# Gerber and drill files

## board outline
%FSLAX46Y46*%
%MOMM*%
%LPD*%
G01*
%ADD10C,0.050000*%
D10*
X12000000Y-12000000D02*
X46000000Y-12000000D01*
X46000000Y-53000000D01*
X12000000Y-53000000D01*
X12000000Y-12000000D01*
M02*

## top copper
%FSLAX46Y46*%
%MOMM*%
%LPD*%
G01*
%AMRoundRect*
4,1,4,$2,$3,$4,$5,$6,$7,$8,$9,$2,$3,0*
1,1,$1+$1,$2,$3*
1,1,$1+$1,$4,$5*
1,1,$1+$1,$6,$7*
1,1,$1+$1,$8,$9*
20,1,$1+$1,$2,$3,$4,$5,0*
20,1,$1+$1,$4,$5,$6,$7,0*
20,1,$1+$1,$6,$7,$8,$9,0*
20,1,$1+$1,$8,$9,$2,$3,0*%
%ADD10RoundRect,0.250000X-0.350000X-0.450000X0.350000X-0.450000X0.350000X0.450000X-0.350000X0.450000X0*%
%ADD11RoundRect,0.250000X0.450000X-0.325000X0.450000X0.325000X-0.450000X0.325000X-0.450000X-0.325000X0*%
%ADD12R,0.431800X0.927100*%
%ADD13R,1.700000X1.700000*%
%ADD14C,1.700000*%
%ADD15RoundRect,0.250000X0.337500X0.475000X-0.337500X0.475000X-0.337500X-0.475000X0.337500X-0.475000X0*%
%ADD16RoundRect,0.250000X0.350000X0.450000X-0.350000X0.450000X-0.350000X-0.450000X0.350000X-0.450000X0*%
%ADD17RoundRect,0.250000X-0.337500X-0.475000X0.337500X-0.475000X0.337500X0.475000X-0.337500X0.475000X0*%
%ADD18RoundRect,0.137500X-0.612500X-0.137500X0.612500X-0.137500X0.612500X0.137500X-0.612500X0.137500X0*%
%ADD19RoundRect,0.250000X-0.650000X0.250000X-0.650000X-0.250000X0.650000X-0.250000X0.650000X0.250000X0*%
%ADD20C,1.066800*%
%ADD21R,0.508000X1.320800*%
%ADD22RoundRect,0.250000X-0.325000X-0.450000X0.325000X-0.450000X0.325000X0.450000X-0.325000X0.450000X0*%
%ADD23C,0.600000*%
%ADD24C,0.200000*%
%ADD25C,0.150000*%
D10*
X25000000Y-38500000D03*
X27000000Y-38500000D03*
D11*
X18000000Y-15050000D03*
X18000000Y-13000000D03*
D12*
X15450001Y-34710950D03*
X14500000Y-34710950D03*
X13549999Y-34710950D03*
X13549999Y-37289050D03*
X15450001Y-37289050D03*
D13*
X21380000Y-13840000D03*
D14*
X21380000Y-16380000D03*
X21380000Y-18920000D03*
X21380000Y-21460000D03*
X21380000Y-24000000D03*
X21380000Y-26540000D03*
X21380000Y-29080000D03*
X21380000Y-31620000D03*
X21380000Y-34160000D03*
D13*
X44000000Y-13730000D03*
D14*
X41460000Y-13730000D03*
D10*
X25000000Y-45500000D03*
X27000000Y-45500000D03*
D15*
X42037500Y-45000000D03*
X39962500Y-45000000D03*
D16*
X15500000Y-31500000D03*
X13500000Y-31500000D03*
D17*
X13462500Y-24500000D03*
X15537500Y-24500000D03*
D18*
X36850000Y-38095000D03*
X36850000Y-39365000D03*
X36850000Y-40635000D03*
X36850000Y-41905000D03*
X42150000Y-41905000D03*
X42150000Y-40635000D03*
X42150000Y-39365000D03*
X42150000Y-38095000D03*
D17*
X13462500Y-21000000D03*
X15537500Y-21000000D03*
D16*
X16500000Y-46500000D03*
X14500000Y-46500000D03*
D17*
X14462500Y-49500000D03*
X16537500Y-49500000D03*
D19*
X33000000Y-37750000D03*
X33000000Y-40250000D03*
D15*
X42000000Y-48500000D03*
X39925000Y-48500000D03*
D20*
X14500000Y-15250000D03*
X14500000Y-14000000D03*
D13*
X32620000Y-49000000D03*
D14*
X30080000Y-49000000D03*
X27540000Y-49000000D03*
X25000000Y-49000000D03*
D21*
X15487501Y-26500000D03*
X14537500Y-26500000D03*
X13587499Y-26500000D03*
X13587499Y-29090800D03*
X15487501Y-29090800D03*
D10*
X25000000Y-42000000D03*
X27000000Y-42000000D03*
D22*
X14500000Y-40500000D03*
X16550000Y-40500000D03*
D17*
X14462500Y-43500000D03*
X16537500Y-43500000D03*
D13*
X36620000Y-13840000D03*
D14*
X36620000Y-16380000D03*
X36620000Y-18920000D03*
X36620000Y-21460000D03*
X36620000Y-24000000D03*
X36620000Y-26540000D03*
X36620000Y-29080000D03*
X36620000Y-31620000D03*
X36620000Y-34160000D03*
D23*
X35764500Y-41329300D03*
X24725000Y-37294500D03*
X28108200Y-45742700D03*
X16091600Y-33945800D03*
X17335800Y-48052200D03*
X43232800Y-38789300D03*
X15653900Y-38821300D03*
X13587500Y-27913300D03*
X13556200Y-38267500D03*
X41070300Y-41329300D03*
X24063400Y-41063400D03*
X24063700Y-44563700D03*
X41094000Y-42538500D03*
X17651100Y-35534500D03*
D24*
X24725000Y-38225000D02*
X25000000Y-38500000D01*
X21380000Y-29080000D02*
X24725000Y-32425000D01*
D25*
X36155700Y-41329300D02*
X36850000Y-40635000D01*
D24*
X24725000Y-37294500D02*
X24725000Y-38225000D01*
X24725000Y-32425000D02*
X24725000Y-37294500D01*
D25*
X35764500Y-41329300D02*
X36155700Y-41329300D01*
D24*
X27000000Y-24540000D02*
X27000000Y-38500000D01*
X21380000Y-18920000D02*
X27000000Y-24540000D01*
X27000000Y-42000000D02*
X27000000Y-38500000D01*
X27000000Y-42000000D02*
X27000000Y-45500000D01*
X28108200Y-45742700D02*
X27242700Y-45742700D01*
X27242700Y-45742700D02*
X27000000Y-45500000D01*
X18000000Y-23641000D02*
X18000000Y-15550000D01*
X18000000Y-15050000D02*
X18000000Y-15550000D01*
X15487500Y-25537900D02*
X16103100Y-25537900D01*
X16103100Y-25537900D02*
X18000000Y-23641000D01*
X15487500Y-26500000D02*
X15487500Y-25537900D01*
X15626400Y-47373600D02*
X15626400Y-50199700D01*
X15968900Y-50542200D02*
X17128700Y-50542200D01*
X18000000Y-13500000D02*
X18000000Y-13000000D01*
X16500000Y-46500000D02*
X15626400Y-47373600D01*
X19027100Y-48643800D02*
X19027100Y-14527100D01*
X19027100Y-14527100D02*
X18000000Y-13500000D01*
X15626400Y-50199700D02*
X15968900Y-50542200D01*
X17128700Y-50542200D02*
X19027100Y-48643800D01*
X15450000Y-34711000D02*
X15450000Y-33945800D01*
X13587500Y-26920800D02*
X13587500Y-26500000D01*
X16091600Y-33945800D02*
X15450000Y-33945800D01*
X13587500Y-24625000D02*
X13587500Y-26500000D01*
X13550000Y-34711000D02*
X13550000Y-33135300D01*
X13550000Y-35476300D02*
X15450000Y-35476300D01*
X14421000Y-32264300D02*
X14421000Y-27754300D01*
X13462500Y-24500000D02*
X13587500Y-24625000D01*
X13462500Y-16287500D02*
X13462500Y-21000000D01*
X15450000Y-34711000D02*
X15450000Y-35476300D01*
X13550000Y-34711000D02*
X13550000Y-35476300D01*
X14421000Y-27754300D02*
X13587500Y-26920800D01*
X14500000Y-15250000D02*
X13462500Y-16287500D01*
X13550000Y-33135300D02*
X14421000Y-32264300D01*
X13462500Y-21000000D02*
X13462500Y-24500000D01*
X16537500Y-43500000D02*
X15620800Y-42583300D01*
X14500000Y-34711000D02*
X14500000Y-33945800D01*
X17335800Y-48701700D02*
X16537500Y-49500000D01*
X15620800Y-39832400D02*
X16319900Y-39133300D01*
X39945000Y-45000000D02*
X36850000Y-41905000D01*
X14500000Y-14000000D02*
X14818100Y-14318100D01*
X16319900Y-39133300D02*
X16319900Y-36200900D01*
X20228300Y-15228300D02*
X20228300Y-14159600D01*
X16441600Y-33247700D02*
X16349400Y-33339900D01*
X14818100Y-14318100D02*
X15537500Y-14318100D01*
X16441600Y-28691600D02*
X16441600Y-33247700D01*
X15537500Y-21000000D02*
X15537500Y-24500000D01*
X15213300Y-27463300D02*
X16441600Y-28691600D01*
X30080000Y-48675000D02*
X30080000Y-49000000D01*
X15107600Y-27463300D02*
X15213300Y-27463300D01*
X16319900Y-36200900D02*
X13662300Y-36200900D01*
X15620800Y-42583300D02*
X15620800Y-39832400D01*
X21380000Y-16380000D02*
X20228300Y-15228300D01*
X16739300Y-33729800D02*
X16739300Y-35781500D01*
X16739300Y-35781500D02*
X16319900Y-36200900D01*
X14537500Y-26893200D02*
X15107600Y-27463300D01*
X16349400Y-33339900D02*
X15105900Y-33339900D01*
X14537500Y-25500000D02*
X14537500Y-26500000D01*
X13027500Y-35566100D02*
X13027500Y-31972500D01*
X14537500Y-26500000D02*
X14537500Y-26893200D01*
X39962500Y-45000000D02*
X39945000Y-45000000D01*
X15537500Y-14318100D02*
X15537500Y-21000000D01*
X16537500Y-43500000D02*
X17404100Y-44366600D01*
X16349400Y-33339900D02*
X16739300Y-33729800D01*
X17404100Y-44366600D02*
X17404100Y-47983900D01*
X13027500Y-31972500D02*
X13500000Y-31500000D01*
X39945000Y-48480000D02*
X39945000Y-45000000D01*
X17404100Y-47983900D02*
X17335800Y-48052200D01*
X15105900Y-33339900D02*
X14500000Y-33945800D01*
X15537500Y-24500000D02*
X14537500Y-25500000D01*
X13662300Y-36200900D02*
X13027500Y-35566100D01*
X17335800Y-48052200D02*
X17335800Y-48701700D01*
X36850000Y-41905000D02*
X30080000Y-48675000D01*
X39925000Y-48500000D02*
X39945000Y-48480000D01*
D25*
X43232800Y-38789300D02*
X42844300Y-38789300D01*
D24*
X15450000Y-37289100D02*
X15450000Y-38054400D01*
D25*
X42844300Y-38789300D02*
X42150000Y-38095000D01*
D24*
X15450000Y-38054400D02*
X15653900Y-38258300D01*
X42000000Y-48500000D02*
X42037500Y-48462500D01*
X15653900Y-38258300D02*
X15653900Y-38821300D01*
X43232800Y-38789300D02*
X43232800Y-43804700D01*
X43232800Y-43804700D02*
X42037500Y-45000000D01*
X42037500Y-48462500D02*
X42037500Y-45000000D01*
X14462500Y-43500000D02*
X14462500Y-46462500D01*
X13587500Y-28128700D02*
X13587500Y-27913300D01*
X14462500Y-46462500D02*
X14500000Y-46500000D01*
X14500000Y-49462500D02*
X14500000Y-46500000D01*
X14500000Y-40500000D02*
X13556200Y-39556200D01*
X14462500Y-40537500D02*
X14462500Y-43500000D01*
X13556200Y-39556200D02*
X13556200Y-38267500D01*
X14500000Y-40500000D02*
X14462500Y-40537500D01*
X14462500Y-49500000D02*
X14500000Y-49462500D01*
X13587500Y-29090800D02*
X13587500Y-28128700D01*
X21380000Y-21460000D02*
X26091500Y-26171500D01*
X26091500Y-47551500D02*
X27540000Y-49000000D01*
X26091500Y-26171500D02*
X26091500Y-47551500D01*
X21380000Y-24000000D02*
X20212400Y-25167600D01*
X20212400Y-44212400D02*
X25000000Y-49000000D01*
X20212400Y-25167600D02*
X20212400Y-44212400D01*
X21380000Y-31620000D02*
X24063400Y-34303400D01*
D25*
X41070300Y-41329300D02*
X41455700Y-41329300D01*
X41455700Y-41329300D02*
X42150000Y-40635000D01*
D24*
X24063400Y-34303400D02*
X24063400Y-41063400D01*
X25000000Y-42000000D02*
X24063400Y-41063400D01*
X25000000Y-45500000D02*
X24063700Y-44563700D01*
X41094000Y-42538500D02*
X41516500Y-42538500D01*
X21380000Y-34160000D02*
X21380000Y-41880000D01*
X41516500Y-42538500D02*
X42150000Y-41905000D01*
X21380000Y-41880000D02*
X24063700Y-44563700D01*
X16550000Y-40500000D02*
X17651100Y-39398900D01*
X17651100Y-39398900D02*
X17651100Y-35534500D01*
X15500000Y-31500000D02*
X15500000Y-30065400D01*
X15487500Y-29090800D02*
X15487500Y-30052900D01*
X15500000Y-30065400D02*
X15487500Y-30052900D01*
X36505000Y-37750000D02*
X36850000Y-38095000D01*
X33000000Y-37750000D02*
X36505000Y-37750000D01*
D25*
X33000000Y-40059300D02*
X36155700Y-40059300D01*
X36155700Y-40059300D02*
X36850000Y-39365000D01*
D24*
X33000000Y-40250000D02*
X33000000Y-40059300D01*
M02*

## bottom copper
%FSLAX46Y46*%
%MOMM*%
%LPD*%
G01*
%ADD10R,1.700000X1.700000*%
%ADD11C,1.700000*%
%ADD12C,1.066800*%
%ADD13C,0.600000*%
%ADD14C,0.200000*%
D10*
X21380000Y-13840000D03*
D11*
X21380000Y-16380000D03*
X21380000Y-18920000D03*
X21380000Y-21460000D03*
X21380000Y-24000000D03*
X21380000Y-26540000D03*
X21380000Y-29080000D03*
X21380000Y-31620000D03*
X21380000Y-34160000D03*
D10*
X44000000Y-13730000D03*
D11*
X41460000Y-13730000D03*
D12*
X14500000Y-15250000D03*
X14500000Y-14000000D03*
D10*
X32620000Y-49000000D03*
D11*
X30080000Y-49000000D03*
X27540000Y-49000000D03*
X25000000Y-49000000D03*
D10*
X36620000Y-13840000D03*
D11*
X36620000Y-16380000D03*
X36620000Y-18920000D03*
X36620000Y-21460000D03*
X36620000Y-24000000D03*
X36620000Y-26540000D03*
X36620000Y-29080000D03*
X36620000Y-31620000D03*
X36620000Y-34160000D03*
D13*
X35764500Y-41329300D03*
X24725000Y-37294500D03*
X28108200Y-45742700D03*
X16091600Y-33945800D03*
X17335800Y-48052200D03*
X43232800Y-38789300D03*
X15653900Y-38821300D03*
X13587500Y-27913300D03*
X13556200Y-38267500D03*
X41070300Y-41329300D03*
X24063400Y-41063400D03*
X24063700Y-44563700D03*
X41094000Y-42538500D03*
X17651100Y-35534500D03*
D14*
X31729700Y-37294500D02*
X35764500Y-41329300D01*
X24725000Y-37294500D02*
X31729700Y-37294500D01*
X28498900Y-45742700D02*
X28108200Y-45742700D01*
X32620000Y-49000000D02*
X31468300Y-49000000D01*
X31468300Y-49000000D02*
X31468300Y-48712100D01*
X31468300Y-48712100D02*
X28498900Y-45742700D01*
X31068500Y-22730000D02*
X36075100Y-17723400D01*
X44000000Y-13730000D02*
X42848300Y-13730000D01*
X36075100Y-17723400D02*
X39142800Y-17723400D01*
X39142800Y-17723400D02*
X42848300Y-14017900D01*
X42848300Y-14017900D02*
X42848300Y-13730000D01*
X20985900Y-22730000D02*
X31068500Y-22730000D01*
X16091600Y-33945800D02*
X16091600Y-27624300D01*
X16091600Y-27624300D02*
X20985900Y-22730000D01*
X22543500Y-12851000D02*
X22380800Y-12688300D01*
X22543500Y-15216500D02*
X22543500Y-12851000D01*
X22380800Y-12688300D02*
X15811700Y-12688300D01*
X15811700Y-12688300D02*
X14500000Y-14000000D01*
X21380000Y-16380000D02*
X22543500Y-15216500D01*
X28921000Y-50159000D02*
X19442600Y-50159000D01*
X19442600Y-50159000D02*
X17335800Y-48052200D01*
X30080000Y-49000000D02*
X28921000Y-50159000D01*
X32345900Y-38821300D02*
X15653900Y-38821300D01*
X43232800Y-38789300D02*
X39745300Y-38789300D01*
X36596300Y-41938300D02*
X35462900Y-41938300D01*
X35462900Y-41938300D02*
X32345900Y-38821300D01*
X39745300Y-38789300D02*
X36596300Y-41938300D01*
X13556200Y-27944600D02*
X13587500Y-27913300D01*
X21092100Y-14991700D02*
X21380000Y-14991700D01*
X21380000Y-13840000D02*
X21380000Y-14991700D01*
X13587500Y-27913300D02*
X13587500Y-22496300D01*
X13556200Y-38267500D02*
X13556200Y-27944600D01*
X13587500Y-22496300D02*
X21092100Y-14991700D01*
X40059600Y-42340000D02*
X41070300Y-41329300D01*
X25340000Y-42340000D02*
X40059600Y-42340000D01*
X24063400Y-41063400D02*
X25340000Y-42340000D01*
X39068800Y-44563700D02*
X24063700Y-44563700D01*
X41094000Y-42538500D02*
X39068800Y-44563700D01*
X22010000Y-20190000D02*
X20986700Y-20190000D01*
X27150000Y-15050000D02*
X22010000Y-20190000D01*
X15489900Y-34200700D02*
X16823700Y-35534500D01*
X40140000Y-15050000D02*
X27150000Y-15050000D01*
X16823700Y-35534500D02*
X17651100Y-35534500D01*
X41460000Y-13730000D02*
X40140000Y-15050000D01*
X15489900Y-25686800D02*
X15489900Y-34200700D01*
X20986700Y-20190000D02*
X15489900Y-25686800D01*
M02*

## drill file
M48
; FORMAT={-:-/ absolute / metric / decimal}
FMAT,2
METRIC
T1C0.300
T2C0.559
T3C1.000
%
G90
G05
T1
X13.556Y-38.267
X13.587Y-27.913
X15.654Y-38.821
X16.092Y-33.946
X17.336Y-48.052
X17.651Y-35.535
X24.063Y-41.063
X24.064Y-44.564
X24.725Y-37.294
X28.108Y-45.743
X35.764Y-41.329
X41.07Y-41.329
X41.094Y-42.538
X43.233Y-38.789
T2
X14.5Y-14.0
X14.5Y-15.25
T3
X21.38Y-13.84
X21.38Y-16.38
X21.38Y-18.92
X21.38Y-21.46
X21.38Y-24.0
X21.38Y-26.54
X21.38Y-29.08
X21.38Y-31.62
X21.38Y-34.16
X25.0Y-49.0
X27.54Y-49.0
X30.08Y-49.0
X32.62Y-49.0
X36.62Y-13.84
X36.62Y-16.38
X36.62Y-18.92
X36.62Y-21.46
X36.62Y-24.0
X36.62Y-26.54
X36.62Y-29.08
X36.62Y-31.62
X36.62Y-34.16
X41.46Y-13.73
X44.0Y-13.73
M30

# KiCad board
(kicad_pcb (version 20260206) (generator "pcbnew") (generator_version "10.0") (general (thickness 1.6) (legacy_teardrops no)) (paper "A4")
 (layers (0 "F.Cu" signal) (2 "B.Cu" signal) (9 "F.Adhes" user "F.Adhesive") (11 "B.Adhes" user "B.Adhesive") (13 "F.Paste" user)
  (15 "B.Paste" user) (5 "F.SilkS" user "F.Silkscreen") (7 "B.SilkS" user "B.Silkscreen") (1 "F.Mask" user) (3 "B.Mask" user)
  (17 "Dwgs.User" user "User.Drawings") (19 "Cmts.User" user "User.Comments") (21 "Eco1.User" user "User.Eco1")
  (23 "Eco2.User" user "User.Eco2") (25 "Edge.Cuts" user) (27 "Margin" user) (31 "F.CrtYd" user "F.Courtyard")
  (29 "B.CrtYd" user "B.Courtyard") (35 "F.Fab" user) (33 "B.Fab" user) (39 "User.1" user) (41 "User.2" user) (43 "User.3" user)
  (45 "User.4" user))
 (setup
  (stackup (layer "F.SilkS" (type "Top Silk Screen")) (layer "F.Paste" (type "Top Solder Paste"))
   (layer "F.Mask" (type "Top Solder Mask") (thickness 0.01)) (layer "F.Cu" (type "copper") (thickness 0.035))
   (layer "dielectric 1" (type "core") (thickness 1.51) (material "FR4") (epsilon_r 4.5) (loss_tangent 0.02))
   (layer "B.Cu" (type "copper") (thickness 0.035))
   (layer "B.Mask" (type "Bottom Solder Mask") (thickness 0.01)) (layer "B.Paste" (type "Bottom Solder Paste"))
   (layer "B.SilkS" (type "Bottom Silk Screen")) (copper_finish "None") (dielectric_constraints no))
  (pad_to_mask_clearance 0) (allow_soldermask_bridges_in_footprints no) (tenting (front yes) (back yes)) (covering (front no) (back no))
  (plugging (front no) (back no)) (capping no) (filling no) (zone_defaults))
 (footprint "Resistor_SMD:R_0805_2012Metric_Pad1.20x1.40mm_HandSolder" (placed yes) (layer "F.Cu") (at 26 38.5)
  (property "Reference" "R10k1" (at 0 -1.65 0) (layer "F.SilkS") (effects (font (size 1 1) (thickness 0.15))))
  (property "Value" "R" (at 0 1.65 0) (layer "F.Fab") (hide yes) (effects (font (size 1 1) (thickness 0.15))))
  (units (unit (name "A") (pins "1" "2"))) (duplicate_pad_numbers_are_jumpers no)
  (pad "1" smd roundrect (at -1 0) (size 1.2 1.4) (layers "F.Cu" "F.Mask" "F.Paste") (roundrect_rratio 0.208333) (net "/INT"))
  (pad "2" smd roundrect (at 1 0) (size 1.2 1.4) (layers "F.Cu" "F.Mask" "F.Paste") (roundrect_rratio 0.208333) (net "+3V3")))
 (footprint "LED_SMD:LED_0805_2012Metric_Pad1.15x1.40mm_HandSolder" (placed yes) (layer "F.Cu") (at 18 14.025 90)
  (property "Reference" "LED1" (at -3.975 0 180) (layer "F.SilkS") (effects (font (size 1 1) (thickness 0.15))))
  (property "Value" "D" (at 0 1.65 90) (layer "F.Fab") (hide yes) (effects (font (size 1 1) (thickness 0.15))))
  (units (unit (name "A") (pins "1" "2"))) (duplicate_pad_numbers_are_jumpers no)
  (pad "1" smd roundrect (at -1.025 0 90) (size 1.15 1.4) (layers "F.Cu" "F.Mask" "F.Paste") (roundrect_rratio 0.217391) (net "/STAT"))
  (pad "2" smd roundrect (at 1.025 0 90) (size 1.15 1.4) (layers "F.Cu" "F.Mask" "F.Paste") (roundrect_rratio 0.217391) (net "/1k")))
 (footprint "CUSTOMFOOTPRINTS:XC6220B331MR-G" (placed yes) (layer "F.Cu") (at 14.5 36 -90)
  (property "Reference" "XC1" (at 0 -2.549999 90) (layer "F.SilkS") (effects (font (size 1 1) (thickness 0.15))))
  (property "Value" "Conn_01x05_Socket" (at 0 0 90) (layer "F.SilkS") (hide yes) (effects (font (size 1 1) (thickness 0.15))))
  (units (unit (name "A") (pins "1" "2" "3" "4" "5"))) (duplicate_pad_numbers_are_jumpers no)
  (pad "1" smd rect (at -1.28905 -0.950001 270) (size 0.9271 0.4318) (layers "F.Cu" "F.Mask" "F.Paste") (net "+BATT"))
  (pad "2" smd rect (at -1.28905 0 270) (size 0.9271 0.4318) (layers "F.Cu" "F.Mask" "F.Paste") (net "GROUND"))
  (pad "3" smd rect (at -1.28905 0.950001 270) (size 0.9271 0.4318) (layers "F.Cu" "F.Mask" "F.Paste") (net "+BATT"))
  (pad "4" smd rect (at 1.28905 0.950001 270) (size 0.9271 0.4318) (layers "F.Cu" "F.Mask" "F.Paste") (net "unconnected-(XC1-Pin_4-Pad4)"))
  (pad "5" smd rect (at 1.28905 -0.950001 270) (size 0.9271 0.4318) (layers "F.Cu" "F.Mask" "F.Paste") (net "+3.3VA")))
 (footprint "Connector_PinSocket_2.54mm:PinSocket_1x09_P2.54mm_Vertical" (layer "F.Cu") (at 21.38 13.84)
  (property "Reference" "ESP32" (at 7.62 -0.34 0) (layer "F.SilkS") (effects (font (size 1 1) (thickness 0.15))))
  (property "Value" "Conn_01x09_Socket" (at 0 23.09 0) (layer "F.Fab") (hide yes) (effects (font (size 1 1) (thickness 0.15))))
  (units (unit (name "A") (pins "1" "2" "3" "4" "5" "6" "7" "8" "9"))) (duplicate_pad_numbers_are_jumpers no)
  (pad "1" thru_hole rect (at 0 0) (size 1.7 1.7) (drill 1) (layers "*.Cu" "*.Mask") (remove_unused_layers no) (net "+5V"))
  (pad "2" thru_hole circle (at 0 2.54) (size 1.7 1.7) (drill 1) (layers "*.Cu" "*.Mask") (remove_unused_layers no) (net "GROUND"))
  (pad "3" thru_hole circle (at 0 5.08) (size 1.7 1.7) (drill 1) (layers "*.Cu" "*.Mask") (remove_unused_layers no) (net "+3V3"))
  (pad "4" thru_hole circle (at 0 7.62) (size 1.7 1.7) (drill 1) (layers "*.Cu" "*.Mask") (remove_unused_layers no) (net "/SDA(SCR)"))
  (pad "5" thru_hole circle (at 0 10.16) (size 1.7 1.7) (drill 1) (layers "*.Cu" "*.Mask") (remove_unused_layers no) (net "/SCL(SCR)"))
  (pad "6" thru_hole circle (at 0 12.7) (size 1.7 1.7) (drill 1) (layers "*.Cu" "*.Mask") (remove_unused_layers no)
   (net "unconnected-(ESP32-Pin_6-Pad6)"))
  (pad "7" thru_hole circle (at 0 15.24) (size 1.7 1.7) (drill 1) (layers "*.Cu" "*.Mask") (remove_unused_layers no) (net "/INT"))
  (pad "8" thru_hole circle (at 0 17.78) (size 1.7 1.7) (drill 1) (layers "*.Cu" "*.Mask") (remove_unused_layers no) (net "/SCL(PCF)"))
  (pad "9" thru_hole circle (at 0 20.32) (size 1.7 1.7) (drill 1) (layers "*.Cu" "*.Mask") (remove_unused_layers no) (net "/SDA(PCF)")))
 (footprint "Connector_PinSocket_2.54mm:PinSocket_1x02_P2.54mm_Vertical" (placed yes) (layer "F.Cu") (at 44 13.73 -90)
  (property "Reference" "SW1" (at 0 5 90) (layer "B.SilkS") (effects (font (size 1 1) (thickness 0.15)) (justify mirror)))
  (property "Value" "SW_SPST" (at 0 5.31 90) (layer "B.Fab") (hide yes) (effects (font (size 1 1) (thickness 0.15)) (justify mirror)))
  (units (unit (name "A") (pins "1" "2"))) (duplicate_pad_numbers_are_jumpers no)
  (pad "1" thru_hole rect (at 0 0 270) (size 1.7 1.7) (drill 1) (layers "*.Cu" "*.Mask") (remove_unused_layers no) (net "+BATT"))
  (pad "2" thru_hole circle (at 0 2.54 270) (size 1.7 1.7) (drill 1) (layers "*.Cu" "*.Mask") (remove_unused_layers no) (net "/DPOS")))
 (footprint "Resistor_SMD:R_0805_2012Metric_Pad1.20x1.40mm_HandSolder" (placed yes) (layer "F.Cu") (at 26 45.5)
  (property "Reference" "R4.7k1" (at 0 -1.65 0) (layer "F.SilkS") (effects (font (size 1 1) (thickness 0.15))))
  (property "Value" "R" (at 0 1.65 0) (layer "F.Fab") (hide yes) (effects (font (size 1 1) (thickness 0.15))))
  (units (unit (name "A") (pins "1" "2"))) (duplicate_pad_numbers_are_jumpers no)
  (pad "1" smd roundrect (at -1 0) (size 1.2 1.4) (layers "F.Cu" "F.Mask" "F.Paste") (roundrect_rratio 0.208333) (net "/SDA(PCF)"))
  (pad "2" smd roundrect (at 1 0) (size 1.2 1.4) (layers "F.Cu" "F.Mask" "F.Paste") (roundrect_rratio 0.208333) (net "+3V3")))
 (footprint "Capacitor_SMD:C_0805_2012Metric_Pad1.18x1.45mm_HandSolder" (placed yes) (layer "F.Cu") (at 41 45 180)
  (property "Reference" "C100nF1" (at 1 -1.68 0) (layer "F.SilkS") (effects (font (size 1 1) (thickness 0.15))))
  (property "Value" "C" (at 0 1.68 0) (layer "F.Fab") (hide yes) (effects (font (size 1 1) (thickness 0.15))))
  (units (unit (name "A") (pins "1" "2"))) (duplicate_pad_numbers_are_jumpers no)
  (pad "1" smd roundrect (at -1.0375 0 180) (size 1.175 1.45) (layers "F.Cu" "F.Mask" "F.Paste") (roundrect_rratio 0.212766) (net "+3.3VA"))
  (pad "2" smd roundrect (at 1.0375 0 180) (size 1.175 1.45) (layers "F.Cu" "F.Mask" "F.Paste") (roundrect_rratio 0.212766) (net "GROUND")))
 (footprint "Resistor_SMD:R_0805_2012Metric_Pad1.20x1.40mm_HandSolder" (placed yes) (layer "F.Cu") (at 14.5 31.5 180)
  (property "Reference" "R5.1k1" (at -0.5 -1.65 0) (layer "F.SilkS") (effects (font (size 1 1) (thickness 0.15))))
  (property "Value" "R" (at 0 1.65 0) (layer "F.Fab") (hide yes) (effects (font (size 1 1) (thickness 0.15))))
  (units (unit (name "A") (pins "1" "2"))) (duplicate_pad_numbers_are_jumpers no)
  (pad "1" smd roundrect (at -1 0 180) (size 1.2 1.4) (layers "F.Cu" "F.Mask" "F.Paste") (roundrect_rratio 0.208333) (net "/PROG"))
  (pad "2" smd roundrect (at 1 0 180) (size 1.2 1.4) (layers "F.Cu" "F.Mask" "F.Paste") (roundrect_rratio 0.208333) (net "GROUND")))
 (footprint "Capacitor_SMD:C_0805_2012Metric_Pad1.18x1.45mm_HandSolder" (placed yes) (layer "F.Cu") (at 14.5 24.5)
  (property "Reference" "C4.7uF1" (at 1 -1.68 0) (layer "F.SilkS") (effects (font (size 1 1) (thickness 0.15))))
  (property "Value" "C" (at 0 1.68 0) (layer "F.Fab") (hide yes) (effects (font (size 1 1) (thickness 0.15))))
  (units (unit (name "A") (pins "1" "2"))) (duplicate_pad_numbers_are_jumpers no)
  (pad "1" smd roundrect (at -1.0375 0) (size 1.175 1.45) (layers "F.Cu" "F.Mask" "F.Paste") (roundrect_rratio 0.212766) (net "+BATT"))
  (pad "2" smd roundrect (at 1.0375 0) (size 1.175 1.45) (layers "F.Cu" "F.Mask" "F.Paste") (roundrect_rratio 0.212766) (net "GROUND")))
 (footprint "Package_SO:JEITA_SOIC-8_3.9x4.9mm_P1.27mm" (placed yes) (layer "F.Cu") (at 39.5 40)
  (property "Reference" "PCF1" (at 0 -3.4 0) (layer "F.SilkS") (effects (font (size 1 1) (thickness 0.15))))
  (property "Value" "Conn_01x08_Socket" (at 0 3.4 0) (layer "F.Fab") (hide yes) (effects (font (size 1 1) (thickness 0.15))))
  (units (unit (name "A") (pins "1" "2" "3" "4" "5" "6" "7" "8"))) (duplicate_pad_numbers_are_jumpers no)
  (pad "1" smd roundrect (at -2.65 -1.905) (size 1.5 0.55) (layers "F.Cu" "F.Mask" "F.Paste") (roundrect_rratio 0.25) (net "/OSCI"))
  (pad "2" smd roundrect (at -2.65 -0.635) (size 1.5 0.55) (layers "F.Cu" "F.Mask" "F.Paste") (roundrect_rratio 0.25) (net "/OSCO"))
  (pad "3" smd roundrect (at -2.65 0.635) (size 1.5 0.55) (layers "F.Cu" "F.Mask" "F.Paste") (roundrect_rratio 0.25) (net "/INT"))
  (pad "4" smd roundrect (at -2.65 1.905) (size 1.5 0.55) (layers "F.Cu" "F.Mask" "F.Paste") (roundrect_rratio 0.25) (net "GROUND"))
  (pad "5" smd roundrect (at 2.65 1.905) (size 1.5 0.55) (layers "F.Cu" "F.Mask" "F.Paste") (roundrect_rratio 0.25) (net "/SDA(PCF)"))
  (pad "6" smd roundrect (at 2.65 0.635) (size 1.5 0.55) (layers "F.Cu" "F.Mask" "F.Paste") (roundrect_rratio 0.25) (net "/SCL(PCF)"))
  (pad "7" smd roundrect (at 2.65 -0.635) (size 1.5 0.55) (layers "F.Cu" "F.Mask" "F.Paste") (roundrect_rratio 0.25)
   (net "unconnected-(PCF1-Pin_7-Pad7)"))
  (pad "8" smd roundrect (at 2.65 -1.905) (size 1.5 0.55) (layers "F.Cu" "F.Mask" "F.Paste") (roundrect_rratio 0.25) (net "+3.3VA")))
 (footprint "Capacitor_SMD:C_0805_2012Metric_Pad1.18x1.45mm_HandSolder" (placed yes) (layer "F.Cu") (at 14.5 21)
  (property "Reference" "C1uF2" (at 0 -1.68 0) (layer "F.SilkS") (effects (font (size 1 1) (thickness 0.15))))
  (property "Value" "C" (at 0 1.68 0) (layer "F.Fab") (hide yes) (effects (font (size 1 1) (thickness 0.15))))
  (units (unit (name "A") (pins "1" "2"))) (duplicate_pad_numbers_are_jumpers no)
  (pad "1" smd roundrect (at -1.0375 0) (size 1.175 1.45) (layers "F.Cu" "F.Mask" "F.Paste") (roundrect_rratio 0.212766) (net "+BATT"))
  (pad "2" smd roundrect (at 1.0375 0) (size 1.175 1.45) (layers "F.Cu" "F.Mask" "F.Paste") (roundrect_rratio 0.212766) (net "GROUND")))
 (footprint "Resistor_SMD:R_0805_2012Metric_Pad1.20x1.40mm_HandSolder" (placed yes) (layer "F.Cu") (at 15.5 46.5 180)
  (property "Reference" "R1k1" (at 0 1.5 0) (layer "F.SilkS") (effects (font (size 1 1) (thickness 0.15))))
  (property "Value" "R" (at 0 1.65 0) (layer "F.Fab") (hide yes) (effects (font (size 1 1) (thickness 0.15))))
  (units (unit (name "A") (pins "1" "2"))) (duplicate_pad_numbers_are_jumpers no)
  (pad "1" smd roundrect (at -1 0 180) (size 1.2 1.4) (layers "F.Cu" "F.Mask" "F.Paste") (roundrect_rratio 0.208333) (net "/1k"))
  (pad "2" smd roundrect (at 1 0 180) (size 1.2 1.4) (layers "F.Cu" "F.Mask" "F.Paste") (roundrect_rratio 0.208333) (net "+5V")))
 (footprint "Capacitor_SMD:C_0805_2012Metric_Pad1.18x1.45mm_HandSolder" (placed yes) (layer "F.Cu") (at 15.5 49.5)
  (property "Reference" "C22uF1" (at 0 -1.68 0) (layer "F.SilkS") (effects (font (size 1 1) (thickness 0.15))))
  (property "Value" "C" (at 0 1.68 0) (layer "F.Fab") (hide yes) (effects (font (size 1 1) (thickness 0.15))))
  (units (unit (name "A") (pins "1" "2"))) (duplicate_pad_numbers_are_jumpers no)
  (pad "1" smd roundrect (at -1.0375 0) (size 1.175 1.45) (layers "F.Cu" "F.Mask" "F.Paste") (roundrect_rratio 0.212766) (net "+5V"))
  (pad "2" smd roundrect (at 1.0375 0) (size 1.175 1.45) (layers "F.Cu" "F.Mask" "F.Paste") (roundrect_rratio 0.212766) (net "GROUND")))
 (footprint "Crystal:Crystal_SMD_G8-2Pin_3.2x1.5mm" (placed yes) (layer "F.Cu") (at 33 39 -90)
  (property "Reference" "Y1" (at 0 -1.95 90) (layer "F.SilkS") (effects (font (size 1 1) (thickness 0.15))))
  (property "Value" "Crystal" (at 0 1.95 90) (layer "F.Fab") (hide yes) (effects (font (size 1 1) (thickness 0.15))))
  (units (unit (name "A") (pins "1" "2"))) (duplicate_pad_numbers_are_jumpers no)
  (pad "1" smd roundrect (at -1.25 0 270) (size 1 1.8) (layers "F.Cu" "F.Mask" "F.Paste") (roundrect_rratio 0.25) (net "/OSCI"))
  (pad "2" smd roundrect (at 1.25 0 270) (size 1 1.8) (layers "F.Cu" "F.Mask" "F.Paste") (roundrect_rratio 0.25) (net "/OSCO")))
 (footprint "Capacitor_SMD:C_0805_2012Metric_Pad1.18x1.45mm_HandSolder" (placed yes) (layer "F.Cu") (at 40.9625 48.5 180)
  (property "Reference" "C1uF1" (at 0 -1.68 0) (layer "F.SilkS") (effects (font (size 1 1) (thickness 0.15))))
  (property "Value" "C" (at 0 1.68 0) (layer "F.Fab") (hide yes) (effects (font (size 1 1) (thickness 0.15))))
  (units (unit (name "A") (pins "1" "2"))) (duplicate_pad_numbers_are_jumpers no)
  (pad "1" smd roundrect (at -1.0375 0 180) (size 1.175 1.45) (layers "F.Cu" "F.Mask" "F.Paste") (roundrect_rratio 0.212766) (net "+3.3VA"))
  (pad "2" smd roundrect (at 1.0375 0 180) (size 1.175 1.45) (layers "F.Cu" "F.Mask" "F.Paste") (roundrect_rratio 0.212766) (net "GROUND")))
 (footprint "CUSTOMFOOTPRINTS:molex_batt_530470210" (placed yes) (layer "F.Cu") (at 14.5 15.25 -90)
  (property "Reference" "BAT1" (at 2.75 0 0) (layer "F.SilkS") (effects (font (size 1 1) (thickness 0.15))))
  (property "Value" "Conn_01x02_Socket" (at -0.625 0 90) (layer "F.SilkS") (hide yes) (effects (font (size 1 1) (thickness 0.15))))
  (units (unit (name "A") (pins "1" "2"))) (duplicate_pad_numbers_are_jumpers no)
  (pad "1" thru_hole circle (at 0 0 270) (size 1.0668 1.0668) (drill 0.5588) (layers "*.Cu" "*.Mask") (remove_unused_layers no)
   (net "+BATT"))
  (pad "2" thru_hole circle (at -1.25 0 270) (size 1.0668 1.0668) (drill 0.5588) (layers "*.Cu" "*.Mask") (remove_unused_layers no)
   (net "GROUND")))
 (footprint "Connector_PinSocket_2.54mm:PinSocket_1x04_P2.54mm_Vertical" (layer "F.Cu") (at 32.62 49 -90)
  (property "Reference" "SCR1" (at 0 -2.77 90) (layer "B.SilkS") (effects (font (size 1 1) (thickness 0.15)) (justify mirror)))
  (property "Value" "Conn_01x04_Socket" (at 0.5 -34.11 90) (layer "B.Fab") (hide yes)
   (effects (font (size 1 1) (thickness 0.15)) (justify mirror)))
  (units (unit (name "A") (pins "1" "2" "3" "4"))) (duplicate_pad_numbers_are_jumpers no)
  (pad "1" thru_hole rect (at 0 0 270) (size 1.7 1.7) (drill 1) (layers "*.Cu" "*.Mask") (remove_unused_layers no) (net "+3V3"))
  (pad "2" thru_hole circle (at 0 2.54 270) (size 1.7 1.7) (drill 1) (layers "*.Cu" "*.Mask") (remove_unused_layers no) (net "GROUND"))
  (pad "3" thru_hole circle (at 0 5.08 270) (size 1.7 1.7) (drill 1) (layers "*.Cu" "*.Mask") (remove_unused_layers no) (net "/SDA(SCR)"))
  (pad "4" thru_hole circle (at 0 7.62 270) (size 1.7 1.7) (drill 1) (layers "*.Cu" "*.Mask") (remove_unused_layers no) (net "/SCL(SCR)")))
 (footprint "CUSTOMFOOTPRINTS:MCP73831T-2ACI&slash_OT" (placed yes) (layer "F.Cu") (at 14.5375 27.7954 -90)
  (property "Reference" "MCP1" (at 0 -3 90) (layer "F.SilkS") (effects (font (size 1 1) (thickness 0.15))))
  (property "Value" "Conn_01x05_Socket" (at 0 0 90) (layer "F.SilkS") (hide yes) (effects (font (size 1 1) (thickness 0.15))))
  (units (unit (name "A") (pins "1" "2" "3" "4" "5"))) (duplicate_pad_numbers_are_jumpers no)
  (pad "1" smd rect (at -1.2954 -0.950001 270) (size 1.3208 0.508) (layers "F.Cu" "F.Mask" "F.Paste") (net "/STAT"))
  (pad "2" smd rect (at -1.2954 0 270) (size 1.3208 0.508) (layers "F.Cu" "F.Mask" "F.Paste") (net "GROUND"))
  (pad "3" smd rect (at -1.2954 0.950001 270) (size 1.3208 0.508) (layers "F.Cu" "F.Mask" "F.Paste") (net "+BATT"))
  (pad "4" smd rect (at 1.2954 0.950001 270) (size 1.3208 0.508) (layers "F.Cu" "F.Mask" "F.Paste") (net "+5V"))
  (pad "5" smd rect (at 1.2954 -0.950001 270) (size 1.3208 0.508) (layers "F.Cu" "F.Mask" "F.Paste") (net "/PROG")))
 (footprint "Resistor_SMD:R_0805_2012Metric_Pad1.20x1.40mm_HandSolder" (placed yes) (layer "F.Cu") (at 26 42)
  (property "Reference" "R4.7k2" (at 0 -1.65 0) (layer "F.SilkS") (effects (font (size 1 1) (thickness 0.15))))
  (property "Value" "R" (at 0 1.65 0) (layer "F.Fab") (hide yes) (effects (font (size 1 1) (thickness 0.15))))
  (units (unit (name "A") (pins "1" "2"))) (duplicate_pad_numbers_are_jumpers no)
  (pad "1" smd roundrect (at -1 0) (size 1.2 1.4) (layers "F.Cu" "F.Mask" "F.Paste") (roundrect_rratio 0.208333) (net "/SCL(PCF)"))
  (pad "2" smd roundrect (at 1 0) (size 1.2 1.4) (layers "F.Cu" "F.Mask" "F.Paste") (roundrect_rratio 0.208333) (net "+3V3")))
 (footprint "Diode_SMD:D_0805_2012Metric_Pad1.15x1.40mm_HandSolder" (layer "F.Cu") (at 15.525 40.5)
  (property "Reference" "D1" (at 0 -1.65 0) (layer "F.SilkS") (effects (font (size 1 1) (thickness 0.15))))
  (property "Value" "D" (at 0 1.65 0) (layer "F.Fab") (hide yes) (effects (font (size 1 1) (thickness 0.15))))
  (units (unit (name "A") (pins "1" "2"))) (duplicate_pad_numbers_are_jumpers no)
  (pad "1" smd roundrect (at -1.025 0) (size 1.15 1.4) (layers "F.Cu" "F.Mask" "F.Paste") (roundrect_rratio 0.217391) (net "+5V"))
  (pad "2" smd roundrect (at 1.025 0) (size 1.15 1.4) (layers "F.Cu" "F.Mask" "F.Paste") (roundrect_rratio 0.217391) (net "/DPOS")))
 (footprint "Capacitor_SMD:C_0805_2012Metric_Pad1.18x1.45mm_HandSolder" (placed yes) (layer "F.Cu") (at 15.5 43.5)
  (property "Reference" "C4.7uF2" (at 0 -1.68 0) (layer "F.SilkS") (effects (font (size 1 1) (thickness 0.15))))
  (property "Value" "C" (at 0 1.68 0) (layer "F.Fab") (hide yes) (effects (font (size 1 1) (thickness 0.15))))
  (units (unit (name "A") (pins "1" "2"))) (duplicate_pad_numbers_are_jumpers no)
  (pad "1" smd roundrect (at -1.0375 0) (size 1.175 1.45) (layers "F.Cu" "F.Mask" "F.Paste") (roundrect_rratio 0.212766) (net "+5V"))
  (pad "2" smd roundrect (at 1.0375 0) (size 1.175 1.45) (layers "F.Cu" "F.Mask" "F.Paste") (roundrect_rratio 0.212766) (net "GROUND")))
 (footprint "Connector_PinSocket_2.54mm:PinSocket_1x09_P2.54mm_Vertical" (layer "F.Cu") (at 36.62 13.84)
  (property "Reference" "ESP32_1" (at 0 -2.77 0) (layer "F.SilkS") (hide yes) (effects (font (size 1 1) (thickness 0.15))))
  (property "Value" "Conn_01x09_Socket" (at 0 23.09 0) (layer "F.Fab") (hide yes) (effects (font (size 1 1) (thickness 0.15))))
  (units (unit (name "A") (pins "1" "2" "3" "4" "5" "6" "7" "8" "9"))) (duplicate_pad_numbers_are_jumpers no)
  (pad "1" thru_hole rect (at 0 0) (size 1.7 1.7) (drill 1) (layers "*.Cu" "*.Mask") (remove_unused_layers no)
   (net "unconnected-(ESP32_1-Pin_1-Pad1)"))
  (pad "2" thru_hole circle (at 0 2.54) (size 1.7 1.7) (drill 1) (layers "*.Cu" "*.Mask") (remove_unused_layers no)
   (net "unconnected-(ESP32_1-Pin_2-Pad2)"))
  (pad "3" thru_hole circle (at 0 5.08) (size 1.7 1.7) (drill 1) (layers "*.Cu" "*.Mask") (remove_unused_layers no)
   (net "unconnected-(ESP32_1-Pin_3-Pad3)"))
  (pad "4" thru_hole circle (at 0 7.62) (size 1.7 1.7) (drill 1) (layers "*.Cu" "*.Mask") (remove_unused_layers no)
   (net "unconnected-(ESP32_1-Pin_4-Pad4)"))
  (pad "5" thru_hole circle (at 0 10.16) (size 1.7 1.7) (drill 1) (layers "*.Cu" "*.Mask") (remove_unused_layers no)
   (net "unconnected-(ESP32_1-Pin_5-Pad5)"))
  (pad "6" thru_hole circle (at 0 12.7) (size 1.7 1.7) (drill 1) (layers "*.Cu" "*.Mask") (remove_unused_layers no)
   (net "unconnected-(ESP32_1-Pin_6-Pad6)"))
  (pad "7" thru_hole circle (at 0 15.24) (size 1.7 1.7) (drill 1) (layers "*.Cu" "*.Mask") (remove_unused_layers no)
   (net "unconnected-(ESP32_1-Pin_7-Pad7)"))
  (pad "8" thru_hole circle (at 0 17.78) (size 1.7 1.7) (drill 1) (layers "*.Cu" "*.Mask") (remove_unused_layers no)
   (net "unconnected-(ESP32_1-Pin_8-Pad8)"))
  (pad "9" thru_hole circle (at 0 20.32) (size 1.7 1.7) (drill 1) (layers "*.Cu" "*.Mask") (remove_unused_layers no)
   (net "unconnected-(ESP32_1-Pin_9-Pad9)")))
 (gr_rect (start 12 12) (end 46 53) (stroke (width 0.05) (type default)) (fill no) (locked yes) (layer "Edge.Cuts"))
 (segment (start 24.725 38.225) (end 25 38.5) (width 0.2) (layer "F.Cu") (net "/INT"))
 (segment (start 21.38 29.08) (end 24.725 32.425) (width 0.2) (layer "F.Cu") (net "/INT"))
 (segment (start 36.1557 41.3293) (end 36.85 40.635) (width 0.15) (layer "F.Cu") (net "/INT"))
 (segment (start 24.725 37.2945) (end 24.725 38.225) (width 0.2) (layer "F.Cu") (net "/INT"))
 (segment (start 24.725 32.425) (end 24.725 37.2945) (width 0.2) (layer "F.Cu") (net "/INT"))
 (segment (start 35.7645 41.3293) (end 36.1557 41.3293) (width 0.15) (layer "F.Cu") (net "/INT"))
 (via (at 35.7645 41.3293) (size 0.6) (drill 0.3) (layers "F.Cu" "B.Cu") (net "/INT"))
 (via (at 24.725 37.2945) (size 0.6) (drill 0.3) (layers "F.Cu" "B.Cu") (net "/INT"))
 (segment (start 31.7297 37.2945) (end 35.7645 41.3293) (width 0.2) (layer "B.Cu") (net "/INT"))
 (segment (start 24.725 37.2945) (end 31.7297 37.2945) (width 0.2) (layer "B.Cu") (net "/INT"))
 (segment (start 27 24.54) (end 27 38.5) (width 0.2) (layer "F.Cu") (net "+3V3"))
 (segment (start 21.38 18.92) (end 27 24.54) (width 0.2) (layer "F.Cu") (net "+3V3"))
 (segment (start 27 42) (end 27 38.5) (width 0.2) (layer "F.Cu") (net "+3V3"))
 (segment (start 27 42) (end 27 45.5) (width 0.2) (layer "F.Cu") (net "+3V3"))
 (segment (start 28.1082 45.7427) (end 27.2427 45.7427) (width 0.2) (layer "F.Cu") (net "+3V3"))
 (segment (start 27.2427 45.7427) (end 27 45.5) (width 0.2) (layer "F.Cu") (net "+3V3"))
 (via (at 28.1082 45.7427) (size 0.6) (drill 0.3) (layers "F.Cu" "B.Cu") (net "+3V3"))
 (segment (start 28.4989 45.7427) (end 28.1082 45.7427) (width 0.2) (layer "B.Cu") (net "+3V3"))
 (segment (start 32.62 49) (end 31.4683 49) (width 0.2) (layer "B.Cu") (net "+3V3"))
 (segment (start 31.4683 49) (end 31.4683 48.7121) (width 0.2) (layer "B.Cu") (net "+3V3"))
 (segment (start 31.4683 48.7121) (end 28.4989 45.7427) (width 0.2) (layer "B.Cu") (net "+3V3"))
 (segment (start 18 23.641) (end 18 15.55) (width 0.2) (layer "F.Cu") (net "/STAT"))
 (segment (start 18 15.05) (end 18 15.55) (width 0.2) (layer "F.Cu") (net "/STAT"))
 (segment (start 15.4875 25.5379) (end 16.1031 25.5379) (width 0.2) (layer "F.Cu") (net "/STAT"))
 (segment (start 16.1031 25.5379) (end 18 23.641) (width 0.2) (layer "F.Cu") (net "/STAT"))
 (segment (start 15.4875 26.5) (end 15.4875 25.5379) (width 0.2) (layer "F.Cu") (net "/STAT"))
 (segment (start 15.6264 47.3736) (end 15.6264 50.1997) (width 0.2) (layer "F.Cu") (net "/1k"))
 (segment (start 15.9689 50.5422) (end 17.1287 50.5422) (width 0.2) (layer "F.Cu") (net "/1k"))
 (segment (start 18 13.5) (end 18 13) (width 0.2) (layer "F.Cu") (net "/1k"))
 (segment (start 16.5 46.5) (end 15.6264 47.3736) (width 0.2) (layer "F.Cu") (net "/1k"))
 (segment (start 19.0271 48.6438) (end 19.0271 14.5271) (width 0.2) (layer "F.Cu") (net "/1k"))
 (segment (start 19.0271 14.5271) (end 18 13.5) (width 0.2) (layer "F.Cu") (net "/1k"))
 (segment (start 15.6264 50.1997) (end 15.9689 50.5422) (width 0.2) (layer "F.Cu") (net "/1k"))
 (segment (start 17.1287 50.5422) (end 19.0271 48.6438) (width 0.2) (layer "F.Cu") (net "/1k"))
 (segment (start 15.45 34.711) (end 15.45 33.9458) (width 0.2) (layer "F.Cu") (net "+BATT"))
 (segment (start 13.5875 26.9208) (end 13.5875 26.5) (width 0.2) (layer "F.Cu") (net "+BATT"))
 (segment (start 16.0916 33.9458) (end 15.45 33.9458) (width 0.2) (layer "F.Cu") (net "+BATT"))
 (segment (start 13.5875 24.625) (end 13.5875 26.5) (width 0.2) (layer "F.Cu") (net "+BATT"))
 (segment (start 13.55 34.711) (end 13.55 33.1353) (width 0.2) (layer "F.Cu") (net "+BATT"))
 (segment (start 13.55 35.4763) (end 15.45 35.4763) (width 0.2) (layer "F.Cu") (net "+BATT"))
 (segment (start 14.421 32.2643) (end 14.421 27.7543) (width 0.2) (layer "F.Cu") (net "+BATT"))
 (segment (start 13.4625 24.5) (end 13.5875 24.625) (width 0.2) (layer "F.Cu") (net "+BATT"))
 (segment (start 13.4625 16.2875) (end 13.4625 21) (width 0.2) (layer "F.Cu") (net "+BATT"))
 (segment (start 15.45 34.711) (end 15.45 35.4763) (width 0.2) (layer "F.Cu") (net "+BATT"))
 (segment (start 13.55 34.711) (end 13.55 35.4763) (width 0.2) (layer "F.Cu") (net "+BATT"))
 (segment (start 14.421 27.7543) (end 13.5875 26.9208) (width 0.2) (layer "F.Cu") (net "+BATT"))
 (segment (start 14.5 15.25) (end 13.4625 16.2875) (width 0.2) (layer "F.Cu") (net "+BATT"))
 (segment (start 13.55 33.1353) (end 14.421 32.2643) (width 0.2) (layer "F.Cu") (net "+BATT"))
 (segment (start 13.4625 21) (end 13.4625 24.5) (width 0.2) (layer "F.Cu") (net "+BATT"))
 (via (at 16.0916 33.9458) (size 0.6) (drill 0.3) (layers "F.Cu" "B.Cu") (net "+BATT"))
 (segment (start 31.0685 22.73) (end 36.0751 17.7234) (width 0.2) (layer "B.Cu") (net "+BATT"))
 (segment (start 44 13.73) (end 42.8483 13.73) (width 0.2) (layer "B.Cu") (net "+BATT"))
 (segment (start 36.0751 17.7234) (end 39.1428 17.7234) (width 0.2) (layer "B.Cu") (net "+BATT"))
 (segment (start 39.1428 17.7234) (end 42.8483 14.0179) (width 0.2) (layer "B.Cu") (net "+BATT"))
 (segment (start 42.8483 14.0179) (end 42.8483 13.73) (width 0.2) (layer "B.Cu") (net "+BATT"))
 (segment (start 20.9859 22.73) (end 31.0685 22.73) (width 0.2) (layer "B.Cu") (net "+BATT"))
 (segment (start 16.0916 33.9458) (end 16.0916 27.6243) (width 0.2) (layer "B.Cu") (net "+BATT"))
 (segment (start 16.0916 27.6243) (end 20.9859 22.73) (width 0.2) (layer "B.Cu") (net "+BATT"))
 (segment (start 16.5375 43.5) (end 15.6208 42.5833) (width 0.2) (layer "F.Cu") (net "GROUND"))
 (segment (start 14.5 34.711) (end 14.5 33.9458) (width 0.2) (layer "F.Cu") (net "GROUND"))
 (segment (start 17.3358 48.7017) (end 16.5375 49.5) (width 0.2) (layer "F.Cu") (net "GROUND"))
 (segment (start 15.6208 39.8324) (end 16.3199 39.1333) (width 0.2) (layer "F.Cu") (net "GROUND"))
 (segment (start 39.945 45) (end 36.85 41.905) (width 0.2) (layer "F.Cu") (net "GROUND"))
 (segment (start 14.5 14) (end 14.8181 14.3181) (width 0.2) (layer "F.Cu") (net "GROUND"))
 (segment (start 16.3199 39.1333) (end 16.3199 36.2009) (width 0.2) (layer "F.Cu") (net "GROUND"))
 (segment (start 20.2283 15.2283) (end 20.2283 14.1596) (width 0.2) (layer "F.Cu") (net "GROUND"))
 (segment (start 16.4416 33.2477) (end 16.3494 33.3399) (width 0.2) (layer "F.Cu") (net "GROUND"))
 (segment (start 14.8181 14.3181) (end 15.5375 14.3181) (width 0.2) (layer "F.Cu") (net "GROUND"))
 (segment (start 16.4416 28.6916) (end 16.4416 33.2477) (width 0.2) (layer "F.Cu") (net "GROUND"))
 (segment (start 15.5375 21) (end 15.5375 24.5) (width 0.2) (layer "F.Cu") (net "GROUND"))
 (segment (start 15.2133 27.4633) (end 16.4416 28.6916) (width 0.2) (layer "F.Cu") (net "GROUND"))
 (segment (start 30.08 48.675) (end 30.08 49) (width 0.2) (layer "F.Cu") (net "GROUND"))
 (segment (start 15.1076 27.4633) (end 15.2133 27.4633) (width 0.2) (layer "F.Cu") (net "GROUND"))
 (segment (start 16.3199 36.2009) (end 13.6623 36.2009) (width 0.2) (layer "F.Cu") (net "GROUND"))
 (segment (start 15.6208 42.5833) (end 15.6208 39.8324) (width 0.2) (layer "F.Cu") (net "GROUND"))
 (segment (start 21.38 16.38) (end 20.2283 15.2283) (width 0.2) (layer "F.Cu") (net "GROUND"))
 (segment (start 16.7393 33.7298) (end 16.7393 35.7815) (width 0.2) (layer "F.Cu") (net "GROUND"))
 (segment (start 16.7393 35.7815) (end 16.3199 36.2009) (width 0.2) (layer "F.Cu") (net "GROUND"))
 (segment (start 14.5375 26.8932) (end 15.1076 27.4633) (width 0.2) (layer "F.Cu") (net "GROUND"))
 (segment (start 16.3494 33.3399) (end 15.1059 33.3399) (width 0.2) (layer "F.Cu") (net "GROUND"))
 (segment (start 14.5375 25.5) (end 14.5375 26.5) (width 0.2) (layer "F.Cu") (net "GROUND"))
 (segment (start 13.0275 35.5661) (end 13.0275 31.9725) (width 0.2) (layer "F.Cu") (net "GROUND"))
 (segment (start 14.5375 26.5) (end 14.5375 26.8932) (width 0.2) (layer "F.Cu") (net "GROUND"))
 (segment (start 39.9625 45) (end 39.945 45) (width 0.2) (layer "F.Cu") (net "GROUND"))
 (segment (start 15.5375 14.3181) (end 15.5375 21) (width 0.2) (layer "F.Cu") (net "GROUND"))
 (segment (start 16.5375 43.5) (end 17.4041 44.3666) (width 0.2) (layer "F.Cu") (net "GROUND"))
 (segment (start 16.3494 33.3399) (end 16.7393 33.7298) (width 0.2) (layer "F.Cu") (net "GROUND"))
 (segment (start 17.4041 44.3666) (end 17.4041 47.9839) (width 0.2) (layer "F.Cu") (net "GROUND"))
 (segment (start 13.0275 31.9725) (end 13.5 31.5) (width 0.2) (layer "F.Cu") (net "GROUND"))
 (segment (start 39.945 48.48) (end 39.945 45) (width 0.2) (layer "F.Cu") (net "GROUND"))
 (segment (start 17.4041 47.9839) (end 17.3358 48.0522) (width 0.2) (layer "F.Cu") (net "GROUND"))
 (segment (start 15.1059 33.3399) (end 14.5 33.9458) (width 0.2) (layer "F.Cu") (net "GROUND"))
 (segment (start 15.5375 24.5) (end 14.5375 25.5) (width 0.2) (layer "F.Cu") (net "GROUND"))
 (segment (start 13.6623 36.2009) (end 13.0275 35.5661) (width 0.2) (layer "F.Cu") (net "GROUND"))
 (segment (start 17.3358 48.0522) (end 17.3358 48.7017) (width 0.2) (layer "F.Cu") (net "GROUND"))
 (segment (start 36.85 41.905) (end 30.08 48.675) (width 0.2) (layer "F.Cu") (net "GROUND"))
 (segment (start 39.925 48.5) (end 39.945 48.48) (width 0.2) (layer "F.Cu") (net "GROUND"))
 (via (at 17.3358 48.0522) (size 0.6) (drill 0.3) (layers "F.Cu" "B.Cu") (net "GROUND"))
 (segment (start 22.5435 12.851) (end 22.3808 12.6883) (width 0.2) (layer "B.Cu") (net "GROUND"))
 (segment (start 22.5435 15.2165) (end 22.5435 12.851) (width 0.2) (layer "B.Cu") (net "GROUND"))
 (segment (start 22.3808 12.6883) (end 15.8117 12.6883) (width 0.2) (layer "B.Cu") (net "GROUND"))
 (segment (start 15.8117 12.6883) (end 14.5 14) (width 0.2) (layer "B.Cu") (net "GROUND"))
 (segment (start 21.38 16.38) (end 22.5435 15.2165) (width 0.2) (layer "B.Cu") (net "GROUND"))
 (segment (start 28.921 50.159) (end 19.4426 50.159) (width 0.2) (layer "B.Cu") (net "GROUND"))
 (segment (start 19.4426 50.159) (end 17.3358 48.0522) (width 0.2) (layer "B.Cu") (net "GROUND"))
 (segment (start 30.08 49) (end 28.921 50.159) (width 0.2) (layer "B.Cu") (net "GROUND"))
 (segment (start 43.2328 38.7893) (end 42.8443 38.7893) (width 0.15) (layer "F.Cu") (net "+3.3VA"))
 (segment (start 15.45 37.2891) (end 15.45 38.0544) (width 0.2) (layer "F.Cu") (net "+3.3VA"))
 (segment (start 42.8443 38.7893) (end 42.15 38.095) (width 0.15) (layer "F.Cu") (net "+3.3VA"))
 (segment (start 15.45 38.0544) (end 15.6539 38.2583) (width 0.2) (layer "F.Cu") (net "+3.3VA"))
 (segment (start 42 48.5) (end 42.0375 48.4625) (width 0.2) (layer "F.Cu") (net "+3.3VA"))
 (segment (start 15.6539 38.2583) (end 15.6539 38.8213) (width 0.2) (layer "F.Cu") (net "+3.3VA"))
 (segment (start 43.2328 38.7893) (end 43.2328 43.8047) (width 0.2) (layer "F.Cu") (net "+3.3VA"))
 (segment (start 43.2328 43.8047) (end 42.0375 45) (width 0.2) (layer "F.Cu") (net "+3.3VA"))
 (segment (start 42.0375 48.4625) (end 42.0375 45) (width 0.2) (layer "F.Cu") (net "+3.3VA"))
 (via (at 43.2328 38.7893) (size 0.6) (drill 0.3) (layers "F.Cu" "B.Cu") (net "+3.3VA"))
 (via (at 15.6539 38.8213) (size 0.6) (drill 0.3) (layers "F.Cu" "B.Cu") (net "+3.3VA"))
 (segment (start 32.3459 38.8213) (end 15.6539 38.8213) (width 0.2) (layer "B.Cu") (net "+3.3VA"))
 (segment (start 43.2328 38.7893) (end 39.7453 38.7893) (width 0.2) (layer "B.Cu") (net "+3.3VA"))
 (segment (start 36.5963 41.9383) (end 35.4629 41.9383) (width 0.2) (layer "B.Cu") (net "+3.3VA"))
 (segment (start 35.4629 41.9383) (end 32.3459 38.8213) (width 0.2) (layer "B.Cu") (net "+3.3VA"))
 (segment (start 39.7453 38.7893) (end 36.5963 41.9383) (width 0.2) (layer "B.Cu") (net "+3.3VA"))
 (segment (start 14.4625 43.5) (end 14.4625 46.4625) (width 0.2) (layer "F.Cu") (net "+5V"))
 (segment (start 13.5875 28.1287) (end 13.5875 27.9133) (width 0.2) (layer "F.Cu") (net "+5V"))
 (segment (start 14.4625 46.4625) (end 14.5 46.5) (width 0.2) (layer "F.Cu") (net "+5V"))
 (segment (start 14.5 49.4625) (end 14.5 46.5) (width 0.2) (layer "F.Cu") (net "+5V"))
 (segment (start 14.5 40.5) (end 13.5562 39.5562) (width 0.2) (layer "F.Cu") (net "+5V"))
 (segment (start 14.4625 40.5375) (end 14.4625 43.5) (width 0.2) (layer "F.Cu") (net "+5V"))
 (segment (start 13.5562 39.5562) (end 13.5562 38.2675) (width 0.2) (layer "F.Cu") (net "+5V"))
 (segment (start 14.5 40.5) (end 14.4625 40.5375) (width 0.2) (layer "F.Cu") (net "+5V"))
 (segment (start 14.4625 49.5) (end 14.5 49.4625) (width 0.2) (layer "F.Cu") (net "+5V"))
 (segment (start 13.5875 29.0908) (end 13.5875 28.1287) (width 0.2) (layer "F.Cu") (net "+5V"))
 (via (at 13.5875 27.9133) (size 0.6) (drill 0.3) (layers "F.Cu" "B.Cu") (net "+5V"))
 (via (at 13.5562 38.2675) (size 0.6) (drill 0.3) (layers "F.Cu" "B.Cu") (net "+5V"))
 (segment (start 13.5562 27.9446) (end 13.5875 27.9133) (width 0.2) (layer "B.Cu") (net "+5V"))
 (segment (start 21.0921 14.9917) (end 21.38 14.9917) (width 0.2) (layer "B.Cu") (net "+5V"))
 (segment (start 21.38 13.84) (end 21.38 14.9917) (width 0.2) (layer "B.Cu") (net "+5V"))
 (segment (start 13.5875 27.9133) (end 13.5875 22.4963) (width 0.2) (layer "B.Cu") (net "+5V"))
 (segment (start 13.5562 38.2675) (end 13.5562 27.9446) (width 0.2) (layer "B.Cu") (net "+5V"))
 (segment (start 13.5875 22.4963) (end 21.0921 14.9917) (width 0.2) (layer "B.Cu") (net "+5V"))
 (segment (start 21.38 21.46) (end 26.0915 26.1715) (width 0.2) (layer "F.Cu") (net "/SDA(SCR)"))
 (segment (start 26.0915 47.5515) (end 27.54 49) (width 0.2) (layer "F.Cu") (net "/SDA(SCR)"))
 (segment (start 26.0915 26.1715) (end 26.0915 47.5515) (width 0.2) (layer "F.Cu") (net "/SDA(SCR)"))
 (segment (start 21.38 24) (end 20.2124 25.1676) (width 0.2) (layer "F.Cu") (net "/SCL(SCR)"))
 (segment (start 20.2124 44.2124) (end 25 49) (width 0.2) (layer "F.Cu") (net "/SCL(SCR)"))
 (segment (start 20.2124 25.1676) (end 20.2124 44.2124) (width 0.2) (layer "F.Cu") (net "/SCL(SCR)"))
 (segment (start 21.38 31.62) (end 24.0634 34.3034) (width 0.2) (layer "F.Cu") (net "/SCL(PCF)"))
 (segment (start 41.0703 41.3293) (end 41.4557 41.3293) (width 0.15) (layer "F.Cu") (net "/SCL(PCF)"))
 (segment (start 41.4557 41.3293) (end 42.15 40.635) (width 0.15) (layer "F.Cu") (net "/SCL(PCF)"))
 (segment (start 24.0634 34.3034) (end 24.0634 41.0634) (width 0.2) (layer "F.Cu") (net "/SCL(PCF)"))
 (segment (start 25 42) (end 24.0634 41.0634) (width 0.2) (layer "F.Cu") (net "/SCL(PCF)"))
 (via (at 41.0703 41.3293) (size 0.6) (drill 0.3) (layers "F.Cu" "B.Cu") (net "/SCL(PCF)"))
 (via (at 24.0634 41.0634) (size 0.6) (drill 0.3) (layers "F.Cu" "B.Cu") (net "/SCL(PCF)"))
 (segment (start 40.0596 42.34) (end 41.0703 41.3293) (width 0.2) (layer "B.Cu") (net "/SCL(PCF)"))
 (segment (start 25.34 42.34) (end 40.0596 42.34) (width 0.2) (layer "B.Cu") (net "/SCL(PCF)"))
 (segment (start 24.0634 41.0634) (end 25.34 42.34) (width 0.2) (layer "B.Cu") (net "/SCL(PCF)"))
 (segment (start 25 45.5) (end 24.0637 44.5637) (width 0.2) (layer "F.Cu") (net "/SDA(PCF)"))
 (segment (start 41.094 42.5385) (end 41.5165 42.5385) (width 0.2) (layer "F.Cu") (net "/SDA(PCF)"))
 (segment (start 21.38 34.16) (end 21.38 41.88) (width 0.2) (layer "F.Cu") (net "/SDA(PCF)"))
 (segment (start 41.5165 42.5385) (end 42.15 41.905) (width 0.2) (layer "F.Cu") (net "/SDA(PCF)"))
 (segment (start 21.38 41.88) (end 24.0637 44.5637) (width 0.2) (layer "F.Cu") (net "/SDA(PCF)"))
 (via (at 24.0637 44.5637) (size 0.6) (drill 0.3) (layers "F.Cu" "B.Cu") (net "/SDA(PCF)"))
 (via (at 41.094 42.5385) (size 0.6) (drill 0.3) (layers "F.Cu" "B.Cu") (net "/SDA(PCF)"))
 (segment (start 39.0688 44.5637) (end 24.0637 44.5637) (width 0.2) (layer "B.Cu") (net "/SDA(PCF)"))
 (segment (start 41.094 42.5385) (end 39.0688 44.5637) (width 0.2) (layer "B.Cu") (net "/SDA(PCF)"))
 (segment (start 16.55 40.5) (end 17.6511 39.3989) (width 0.2) (layer "F.Cu") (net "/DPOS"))
 (segment (start 17.6511 39.3989) (end 17.6511 35.5345) (width 0.2) (layer "F.Cu") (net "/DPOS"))
 (via (at 17.6511 35.5345) (size 0.6) (drill 0.3) (layers "F.Cu" "B.Cu") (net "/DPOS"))
 (segment (start 22.01 20.19) (end 20.9867 20.19) (width 0.2) (layer "B.Cu") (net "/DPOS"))
 (segment (start 27.15 15.05) (end 22.01 20.19) (width 0.2) (layer "B.Cu") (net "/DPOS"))
 (segment (start 15.4899 34.2007) (end 16.8237 35.5345) (width 0.2) (layer "B.Cu") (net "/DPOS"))
 (segment (start 40.14 15.05) (end 27.15 15.05) (width 0.2) (layer "B.Cu") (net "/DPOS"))
 (segment (start 16.8237 35.5345) (end 17.6511 35.5345) (width 0.2) (layer "B.Cu") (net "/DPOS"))
 (segment (start 41.46 13.73) (end 40.14 15.05) (width 0.2) (layer "B.Cu") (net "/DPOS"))
 (segment (start 15.4899 25.6868) (end 15.4899 34.2007) (width 0.2) (layer "B.Cu") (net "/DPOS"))
 (segment (start 20.9867 20.19) (end 15.4899 25.6868) (width 0.2) (layer "B.Cu") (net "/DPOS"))
 (segment (start 15.5 31.5) (end 15.5 30.0654) (width 0.2) (layer "F.Cu") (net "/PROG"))
 (segment (start 15.4875 29.0908) (end 15.4875 30.0529) (width 0.2) (layer "F.Cu") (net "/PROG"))
 (segment (start 15.5 30.0654) (end 15.4875 30.0529) (width 0.2) (layer "F.Cu") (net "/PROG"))
 (segment (start 36.505 37.75) (end 36.85 38.095) (width 0.2) (layer "F.Cu") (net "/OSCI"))
 (segment (start 33 37.75) (end 36.505 37.75) (width 0.2) (layer "F.Cu") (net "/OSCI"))
 (segment (start 33 40.0593) (end 36.1557 40.0593) (width 0.15) (layer "F.Cu") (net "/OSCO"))
 (segment (start 36.1557 40.0593) (end 36.85 39.365) (width 0.15) (layer "F.Cu") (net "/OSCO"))
 (segment (start 33 40.25) (end 33 40.0593) (width 0.2) (layer "F.Cu") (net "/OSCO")))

